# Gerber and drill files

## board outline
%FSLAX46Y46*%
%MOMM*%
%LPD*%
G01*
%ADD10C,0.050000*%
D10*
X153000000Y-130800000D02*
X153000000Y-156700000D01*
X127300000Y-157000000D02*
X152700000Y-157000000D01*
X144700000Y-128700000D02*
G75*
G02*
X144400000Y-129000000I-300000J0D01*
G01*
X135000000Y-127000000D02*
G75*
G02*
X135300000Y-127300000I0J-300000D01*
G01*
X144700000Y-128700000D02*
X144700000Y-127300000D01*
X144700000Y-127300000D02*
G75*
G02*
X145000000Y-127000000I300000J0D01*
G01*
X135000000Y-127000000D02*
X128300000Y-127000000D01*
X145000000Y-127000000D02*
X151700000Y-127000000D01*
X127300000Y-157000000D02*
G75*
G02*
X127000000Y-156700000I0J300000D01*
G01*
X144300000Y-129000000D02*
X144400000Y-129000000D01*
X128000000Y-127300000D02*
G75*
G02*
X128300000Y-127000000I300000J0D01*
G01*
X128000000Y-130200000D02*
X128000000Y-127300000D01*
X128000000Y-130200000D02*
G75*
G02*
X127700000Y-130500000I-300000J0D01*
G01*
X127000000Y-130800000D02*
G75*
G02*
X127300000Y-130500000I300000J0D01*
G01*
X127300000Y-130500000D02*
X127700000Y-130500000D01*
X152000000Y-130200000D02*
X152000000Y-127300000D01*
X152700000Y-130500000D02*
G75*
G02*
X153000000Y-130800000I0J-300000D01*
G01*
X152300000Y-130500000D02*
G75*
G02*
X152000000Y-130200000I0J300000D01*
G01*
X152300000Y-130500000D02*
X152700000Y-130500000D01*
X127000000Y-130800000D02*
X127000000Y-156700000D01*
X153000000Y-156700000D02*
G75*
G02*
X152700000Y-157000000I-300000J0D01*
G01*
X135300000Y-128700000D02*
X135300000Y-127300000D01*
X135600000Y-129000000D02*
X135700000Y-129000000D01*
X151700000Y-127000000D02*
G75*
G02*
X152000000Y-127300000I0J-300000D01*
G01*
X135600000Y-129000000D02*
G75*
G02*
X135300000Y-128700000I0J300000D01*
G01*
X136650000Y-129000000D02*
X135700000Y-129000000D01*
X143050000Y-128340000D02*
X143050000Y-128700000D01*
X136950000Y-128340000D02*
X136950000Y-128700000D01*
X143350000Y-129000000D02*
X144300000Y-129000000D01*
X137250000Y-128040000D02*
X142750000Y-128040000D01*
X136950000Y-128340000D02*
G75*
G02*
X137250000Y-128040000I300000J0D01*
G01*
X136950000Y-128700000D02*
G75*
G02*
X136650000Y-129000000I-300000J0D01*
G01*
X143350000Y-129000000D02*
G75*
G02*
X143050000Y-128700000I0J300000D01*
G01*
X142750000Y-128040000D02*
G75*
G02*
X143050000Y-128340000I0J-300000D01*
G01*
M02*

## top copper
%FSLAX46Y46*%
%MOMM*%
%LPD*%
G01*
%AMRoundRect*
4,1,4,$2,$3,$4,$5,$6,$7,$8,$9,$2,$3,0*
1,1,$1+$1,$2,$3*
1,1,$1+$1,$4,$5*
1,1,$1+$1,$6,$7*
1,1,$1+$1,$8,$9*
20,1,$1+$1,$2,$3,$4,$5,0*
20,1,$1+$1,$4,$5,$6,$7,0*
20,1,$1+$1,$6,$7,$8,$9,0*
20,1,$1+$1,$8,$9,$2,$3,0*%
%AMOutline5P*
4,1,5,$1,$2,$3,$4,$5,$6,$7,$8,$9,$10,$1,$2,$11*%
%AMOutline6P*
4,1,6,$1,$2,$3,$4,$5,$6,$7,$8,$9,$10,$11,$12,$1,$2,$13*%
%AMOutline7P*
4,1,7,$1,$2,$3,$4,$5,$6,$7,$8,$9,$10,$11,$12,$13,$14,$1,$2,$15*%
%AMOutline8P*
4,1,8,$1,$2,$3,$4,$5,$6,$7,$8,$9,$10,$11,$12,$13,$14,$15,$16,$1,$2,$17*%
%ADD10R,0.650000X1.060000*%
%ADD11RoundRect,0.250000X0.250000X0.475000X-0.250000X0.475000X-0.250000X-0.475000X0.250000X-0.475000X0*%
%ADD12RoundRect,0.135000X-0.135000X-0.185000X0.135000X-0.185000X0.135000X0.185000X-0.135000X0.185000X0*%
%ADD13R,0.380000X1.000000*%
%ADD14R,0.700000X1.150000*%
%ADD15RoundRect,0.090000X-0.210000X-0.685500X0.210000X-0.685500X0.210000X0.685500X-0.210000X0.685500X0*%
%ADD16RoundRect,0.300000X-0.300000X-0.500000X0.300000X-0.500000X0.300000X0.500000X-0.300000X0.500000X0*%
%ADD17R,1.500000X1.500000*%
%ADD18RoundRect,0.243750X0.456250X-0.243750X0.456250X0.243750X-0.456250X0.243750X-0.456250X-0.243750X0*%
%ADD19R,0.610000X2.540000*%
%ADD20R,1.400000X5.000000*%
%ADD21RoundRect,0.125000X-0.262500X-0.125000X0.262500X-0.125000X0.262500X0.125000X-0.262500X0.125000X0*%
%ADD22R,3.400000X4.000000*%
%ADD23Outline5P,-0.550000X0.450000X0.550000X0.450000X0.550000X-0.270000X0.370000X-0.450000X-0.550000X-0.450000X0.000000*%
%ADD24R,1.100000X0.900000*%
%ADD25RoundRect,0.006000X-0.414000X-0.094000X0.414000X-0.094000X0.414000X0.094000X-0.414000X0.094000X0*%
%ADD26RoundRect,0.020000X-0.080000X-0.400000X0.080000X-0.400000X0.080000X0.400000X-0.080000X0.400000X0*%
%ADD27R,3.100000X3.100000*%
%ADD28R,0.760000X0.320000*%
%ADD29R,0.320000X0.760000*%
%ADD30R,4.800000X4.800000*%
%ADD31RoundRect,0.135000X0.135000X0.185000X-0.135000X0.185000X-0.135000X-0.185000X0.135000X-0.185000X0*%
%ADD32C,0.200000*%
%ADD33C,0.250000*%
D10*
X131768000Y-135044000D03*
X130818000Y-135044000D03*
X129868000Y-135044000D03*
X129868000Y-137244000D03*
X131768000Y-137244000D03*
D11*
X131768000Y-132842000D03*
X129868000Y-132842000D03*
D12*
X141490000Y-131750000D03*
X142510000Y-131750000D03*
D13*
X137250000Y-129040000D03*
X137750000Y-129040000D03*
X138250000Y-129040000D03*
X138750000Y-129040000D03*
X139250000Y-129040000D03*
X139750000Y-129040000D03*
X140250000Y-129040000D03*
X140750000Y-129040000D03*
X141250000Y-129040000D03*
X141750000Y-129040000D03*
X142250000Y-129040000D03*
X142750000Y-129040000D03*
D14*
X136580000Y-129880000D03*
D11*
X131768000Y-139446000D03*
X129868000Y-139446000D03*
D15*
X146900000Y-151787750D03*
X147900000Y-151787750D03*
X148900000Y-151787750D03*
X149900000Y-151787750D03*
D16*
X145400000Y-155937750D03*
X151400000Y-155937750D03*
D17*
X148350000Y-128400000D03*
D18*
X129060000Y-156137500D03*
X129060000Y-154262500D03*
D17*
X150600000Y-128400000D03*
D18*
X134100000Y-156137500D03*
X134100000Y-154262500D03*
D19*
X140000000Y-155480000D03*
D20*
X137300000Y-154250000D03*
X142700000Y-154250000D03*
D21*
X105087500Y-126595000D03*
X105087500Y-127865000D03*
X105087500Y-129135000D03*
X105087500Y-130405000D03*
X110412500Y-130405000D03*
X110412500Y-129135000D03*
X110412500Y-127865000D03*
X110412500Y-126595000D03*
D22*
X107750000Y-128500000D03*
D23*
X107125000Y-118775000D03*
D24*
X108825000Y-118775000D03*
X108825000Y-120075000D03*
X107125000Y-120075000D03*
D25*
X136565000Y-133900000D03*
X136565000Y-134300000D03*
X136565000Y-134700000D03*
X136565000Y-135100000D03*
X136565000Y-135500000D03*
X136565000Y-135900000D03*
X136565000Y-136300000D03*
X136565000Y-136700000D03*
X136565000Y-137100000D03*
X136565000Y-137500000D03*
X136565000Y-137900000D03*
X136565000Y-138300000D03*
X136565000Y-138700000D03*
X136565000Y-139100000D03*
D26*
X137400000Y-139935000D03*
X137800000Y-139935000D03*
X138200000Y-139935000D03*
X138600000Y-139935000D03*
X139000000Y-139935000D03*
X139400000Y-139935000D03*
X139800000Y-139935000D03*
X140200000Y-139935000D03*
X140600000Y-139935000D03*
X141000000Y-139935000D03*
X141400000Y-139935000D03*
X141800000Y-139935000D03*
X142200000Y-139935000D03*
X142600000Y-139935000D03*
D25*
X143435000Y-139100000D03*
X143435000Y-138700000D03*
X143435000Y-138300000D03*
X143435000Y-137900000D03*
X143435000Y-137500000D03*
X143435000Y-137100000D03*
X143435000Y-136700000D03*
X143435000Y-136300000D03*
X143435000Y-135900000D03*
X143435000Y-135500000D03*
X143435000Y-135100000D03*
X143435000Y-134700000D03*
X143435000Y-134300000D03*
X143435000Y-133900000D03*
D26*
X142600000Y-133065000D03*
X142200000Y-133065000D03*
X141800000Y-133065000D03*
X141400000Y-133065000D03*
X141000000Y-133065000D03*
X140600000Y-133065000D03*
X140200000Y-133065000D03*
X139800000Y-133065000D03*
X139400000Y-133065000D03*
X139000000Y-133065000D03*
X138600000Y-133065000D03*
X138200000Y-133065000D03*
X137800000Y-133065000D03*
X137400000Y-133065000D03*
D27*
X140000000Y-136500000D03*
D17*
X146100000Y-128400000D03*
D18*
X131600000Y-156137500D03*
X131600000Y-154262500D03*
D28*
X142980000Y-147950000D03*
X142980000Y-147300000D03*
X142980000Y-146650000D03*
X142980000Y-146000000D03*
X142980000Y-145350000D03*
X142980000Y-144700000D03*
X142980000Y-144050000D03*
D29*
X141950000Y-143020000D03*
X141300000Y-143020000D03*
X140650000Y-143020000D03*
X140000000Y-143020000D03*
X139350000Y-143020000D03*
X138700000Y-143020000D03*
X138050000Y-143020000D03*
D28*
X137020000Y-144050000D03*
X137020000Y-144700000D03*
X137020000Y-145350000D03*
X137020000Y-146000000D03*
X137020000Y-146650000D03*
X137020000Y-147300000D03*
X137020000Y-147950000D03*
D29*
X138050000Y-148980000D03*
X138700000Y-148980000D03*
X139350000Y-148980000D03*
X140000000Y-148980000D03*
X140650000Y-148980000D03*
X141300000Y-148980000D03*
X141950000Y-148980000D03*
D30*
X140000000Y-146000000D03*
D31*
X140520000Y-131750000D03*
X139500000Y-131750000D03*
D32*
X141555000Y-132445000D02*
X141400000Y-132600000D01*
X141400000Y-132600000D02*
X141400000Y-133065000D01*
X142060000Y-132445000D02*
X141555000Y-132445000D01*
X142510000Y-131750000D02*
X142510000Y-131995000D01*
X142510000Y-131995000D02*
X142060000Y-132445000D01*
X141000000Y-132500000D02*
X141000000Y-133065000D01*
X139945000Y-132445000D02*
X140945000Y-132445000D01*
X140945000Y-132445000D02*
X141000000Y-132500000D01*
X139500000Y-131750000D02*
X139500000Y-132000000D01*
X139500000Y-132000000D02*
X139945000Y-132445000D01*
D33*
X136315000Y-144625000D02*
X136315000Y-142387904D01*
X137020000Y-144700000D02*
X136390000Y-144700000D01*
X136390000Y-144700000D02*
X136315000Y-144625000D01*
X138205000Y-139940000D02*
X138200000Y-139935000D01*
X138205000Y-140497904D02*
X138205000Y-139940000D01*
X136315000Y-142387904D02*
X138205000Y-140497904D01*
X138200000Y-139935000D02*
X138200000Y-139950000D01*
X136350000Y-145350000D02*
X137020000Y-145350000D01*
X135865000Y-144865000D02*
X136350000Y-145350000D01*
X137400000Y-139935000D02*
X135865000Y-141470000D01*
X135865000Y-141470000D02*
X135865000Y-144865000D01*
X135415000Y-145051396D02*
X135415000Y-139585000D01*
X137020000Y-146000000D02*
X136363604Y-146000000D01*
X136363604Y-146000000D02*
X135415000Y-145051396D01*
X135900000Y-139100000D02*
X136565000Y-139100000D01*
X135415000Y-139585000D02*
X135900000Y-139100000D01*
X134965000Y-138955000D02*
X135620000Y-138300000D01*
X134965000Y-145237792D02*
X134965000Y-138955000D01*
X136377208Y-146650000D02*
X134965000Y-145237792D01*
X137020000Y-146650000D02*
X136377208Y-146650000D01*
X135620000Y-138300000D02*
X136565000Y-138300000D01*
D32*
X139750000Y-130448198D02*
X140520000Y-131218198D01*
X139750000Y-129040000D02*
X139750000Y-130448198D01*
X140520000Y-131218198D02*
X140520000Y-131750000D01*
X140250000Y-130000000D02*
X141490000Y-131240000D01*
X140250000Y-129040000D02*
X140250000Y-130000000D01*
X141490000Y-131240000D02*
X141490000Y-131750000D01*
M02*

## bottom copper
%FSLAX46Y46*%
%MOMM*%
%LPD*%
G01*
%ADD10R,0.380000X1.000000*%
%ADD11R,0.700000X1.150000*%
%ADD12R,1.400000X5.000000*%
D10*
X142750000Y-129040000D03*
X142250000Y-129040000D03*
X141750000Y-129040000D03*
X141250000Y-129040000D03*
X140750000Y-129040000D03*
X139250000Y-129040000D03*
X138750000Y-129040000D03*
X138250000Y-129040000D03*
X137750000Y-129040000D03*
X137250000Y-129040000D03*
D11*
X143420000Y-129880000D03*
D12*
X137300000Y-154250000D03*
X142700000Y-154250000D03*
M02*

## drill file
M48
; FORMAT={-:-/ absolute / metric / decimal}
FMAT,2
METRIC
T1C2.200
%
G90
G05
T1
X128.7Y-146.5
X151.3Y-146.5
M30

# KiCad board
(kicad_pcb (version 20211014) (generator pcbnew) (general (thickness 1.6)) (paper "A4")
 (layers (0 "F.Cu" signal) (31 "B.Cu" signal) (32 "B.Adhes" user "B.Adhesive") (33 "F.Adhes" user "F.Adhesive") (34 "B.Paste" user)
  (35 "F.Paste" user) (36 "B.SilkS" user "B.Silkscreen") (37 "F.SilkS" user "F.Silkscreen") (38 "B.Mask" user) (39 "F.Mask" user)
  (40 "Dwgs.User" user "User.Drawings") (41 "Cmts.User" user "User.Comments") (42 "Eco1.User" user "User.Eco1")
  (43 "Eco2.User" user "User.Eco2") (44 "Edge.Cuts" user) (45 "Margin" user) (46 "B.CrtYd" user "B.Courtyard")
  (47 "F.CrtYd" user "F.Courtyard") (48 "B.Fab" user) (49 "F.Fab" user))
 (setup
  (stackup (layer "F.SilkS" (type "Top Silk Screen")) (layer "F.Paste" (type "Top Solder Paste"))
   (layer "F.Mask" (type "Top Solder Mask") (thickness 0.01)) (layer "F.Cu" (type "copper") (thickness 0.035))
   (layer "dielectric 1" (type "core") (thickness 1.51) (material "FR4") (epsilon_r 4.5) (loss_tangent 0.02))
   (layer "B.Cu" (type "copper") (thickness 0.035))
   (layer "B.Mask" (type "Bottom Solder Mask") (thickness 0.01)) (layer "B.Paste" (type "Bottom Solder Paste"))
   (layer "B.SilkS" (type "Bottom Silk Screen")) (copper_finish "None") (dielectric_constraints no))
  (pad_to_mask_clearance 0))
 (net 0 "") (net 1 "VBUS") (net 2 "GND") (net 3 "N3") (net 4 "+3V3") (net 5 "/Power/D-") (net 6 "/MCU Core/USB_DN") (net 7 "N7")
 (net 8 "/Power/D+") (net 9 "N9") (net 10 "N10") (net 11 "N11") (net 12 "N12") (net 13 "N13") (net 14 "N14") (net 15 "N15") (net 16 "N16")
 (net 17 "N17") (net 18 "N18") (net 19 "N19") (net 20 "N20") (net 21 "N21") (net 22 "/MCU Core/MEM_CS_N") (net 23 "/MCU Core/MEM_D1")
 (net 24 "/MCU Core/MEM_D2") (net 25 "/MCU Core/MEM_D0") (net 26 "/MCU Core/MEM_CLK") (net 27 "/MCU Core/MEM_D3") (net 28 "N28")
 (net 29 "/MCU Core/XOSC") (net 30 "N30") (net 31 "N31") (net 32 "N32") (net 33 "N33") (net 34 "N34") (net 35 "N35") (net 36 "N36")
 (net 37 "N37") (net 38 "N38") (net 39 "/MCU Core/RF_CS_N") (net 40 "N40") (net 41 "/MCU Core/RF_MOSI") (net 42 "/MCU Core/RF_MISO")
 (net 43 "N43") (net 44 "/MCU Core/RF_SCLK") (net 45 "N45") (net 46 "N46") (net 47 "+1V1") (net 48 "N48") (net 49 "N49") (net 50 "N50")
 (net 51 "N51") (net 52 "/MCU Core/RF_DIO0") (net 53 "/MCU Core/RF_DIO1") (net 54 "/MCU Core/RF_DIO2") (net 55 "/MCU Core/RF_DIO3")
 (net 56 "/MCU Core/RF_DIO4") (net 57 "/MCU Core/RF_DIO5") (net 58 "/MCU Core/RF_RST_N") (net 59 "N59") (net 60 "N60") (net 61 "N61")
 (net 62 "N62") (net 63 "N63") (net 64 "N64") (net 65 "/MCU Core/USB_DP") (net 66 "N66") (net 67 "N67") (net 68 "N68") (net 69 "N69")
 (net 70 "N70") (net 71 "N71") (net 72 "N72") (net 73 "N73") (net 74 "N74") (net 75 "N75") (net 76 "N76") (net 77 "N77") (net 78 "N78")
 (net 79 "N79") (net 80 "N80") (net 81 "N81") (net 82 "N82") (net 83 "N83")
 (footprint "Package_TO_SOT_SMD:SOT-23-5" (layer "F.Cu") (at 130.818 136.144 -90)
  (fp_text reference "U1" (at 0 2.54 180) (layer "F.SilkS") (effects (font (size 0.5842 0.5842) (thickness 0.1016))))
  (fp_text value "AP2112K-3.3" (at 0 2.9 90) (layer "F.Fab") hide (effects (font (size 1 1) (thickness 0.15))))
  (pad "1" smd rect locked (at -1.1 -0.95 270) (size 1.06 0.65) (layers "F.Cu" "F.Paste" "F.Mask") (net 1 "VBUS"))
  (pad "2" smd rect locked (at -1.1 0 270) (size 1.06 0.65) (layers "F.Cu" "F.Paste" "F.Mask") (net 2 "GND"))
  (pad "3" smd rect locked (at -1.1 0.95 270) (size 1.06 0.65) (layers "F.Cu" "F.Paste" "F.Mask") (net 1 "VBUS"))
  (pad "4" smd rect locked (at 1.1 0.95 270) (size 1.06 0.65) (layers "F.Cu" "F.Paste" "F.Mask") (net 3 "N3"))
  (pad "5" smd rect locked (at 1.1 -0.95 270) (size 1.06 0.65) (layers "F.Cu" "F.Paste" "F.Mask") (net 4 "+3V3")))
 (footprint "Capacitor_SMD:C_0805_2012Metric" (layer "F.Cu") (at 130.818 132.842 180)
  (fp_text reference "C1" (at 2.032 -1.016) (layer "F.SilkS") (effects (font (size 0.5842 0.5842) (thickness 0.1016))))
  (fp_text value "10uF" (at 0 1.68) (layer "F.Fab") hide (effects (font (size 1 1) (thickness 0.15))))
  (pad "1" smd roundrect locked (at -0.95 0 180) (size 1 1.45) (layers "F.Cu" "F.Paste" "F.Mask") (roundrect_rratio 0.25) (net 1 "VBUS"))
  (pad "2" smd roundrect locked (at 0.95 0 180) (size 1 1.45) (layers "F.Cu" "F.Paste" "F.Mask") (roundrect_rratio 0.25) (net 2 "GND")))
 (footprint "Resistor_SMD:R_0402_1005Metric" (layer "F.Cu") (at 142 131.75)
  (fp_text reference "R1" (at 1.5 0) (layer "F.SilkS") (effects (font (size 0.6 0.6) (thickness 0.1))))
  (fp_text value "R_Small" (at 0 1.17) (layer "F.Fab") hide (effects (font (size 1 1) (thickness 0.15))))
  (pad "1" smd roundrect (at -0.51 0) (size 0.54 0.64) (layers "F.Cu" "F.Paste" "F.Mask") (roundrect_rratio 0.25) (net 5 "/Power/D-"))
  (pad "2" smd roundrect (at 0.51 0) (size 0.54 0.64) (layers "F.Cu" "F.Paste" "F.Mask") (roundrect_rratio 0.25) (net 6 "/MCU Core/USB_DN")))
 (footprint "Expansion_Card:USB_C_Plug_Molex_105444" (layer "F.Cu") (at 140 129) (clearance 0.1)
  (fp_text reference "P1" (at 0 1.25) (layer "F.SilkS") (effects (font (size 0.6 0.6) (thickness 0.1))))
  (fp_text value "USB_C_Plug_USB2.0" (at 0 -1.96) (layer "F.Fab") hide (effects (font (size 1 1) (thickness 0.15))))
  (fp_line (start -3.35 0) (end -4.3 0) (layer "Edge.Cuts") (width 0.05))
  (fp_line (start 3.05 -0.66) (end 3.05 -0.3) (layer "Edge.Cuts") (width 0.05))
  (fp_line (start -3.05 -0.66) (end -3.05 -0.3) (layer "Edge.Cuts") (width 0.05))
  (fp_line (start 3.35 0) (end 4.3 0) (layer "Edge.Cuts") (width 0.05))
  (fp_line (start -2.75 -0.96) (end 2.75 -0.96) (layer "Edge.Cuts") (width 0.05))
  (fp_arc (start -3.05 -0.66) (mid -2.962132 -0.872132) (end -2.75 -0.96) (layer "Edge.Cuts") (width 0.05))
  (fp_arc (start -3.05 -0.3) (mid -3.137868 -0.087868) (end -3.35 0) (layer "Edge.Cuts") (width 0.05))
  (fp_arc (start 3.35 0) (mid 3.137868 -0.087868) (end 3.05 -0.3) (layer "Edge.Cuts") (width 0.05))
  (fp_arc (start 2.75 -0.96) (mid 2.962132 -0.872132) (end 3.05 -0.66) (layer "Edge.Cuts") (width 0.05))
  (pad "A1" smd rect locked (at -2.75 0.04) (size 0.38 1) (layers "F.Cu" "F.Paste" "F.Mask") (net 2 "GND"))
  (pad "A2" smd rect locked (at -2.25 0.04) (size 0.38 1) (layers "F.Cu" "F.Paste" "F.Mask"))
  (pad "A3" smd rect locked (at -1.75 0.04) (size 0.38 1) (layers "F.Cu" "F.Paste" "F.Mask"))
  (pad "A4" smd rect locked (at -1.25 0.04) (size 0.38 1) (layers "F.Cu" "F.Paste" "F.Mask") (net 1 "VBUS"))
  (pad "A5" smd rect locked (at -0.75 0.04) (size 0.38 1) (layers "F.Cu" "F.Paste" "F.Mask") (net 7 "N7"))
  (pad "A6" smd rect locked (at -0.25 0.04) (size 0.38 1) (layers "F.Cu" "F.Paste" "F.Mask") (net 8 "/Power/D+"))
  (pad "A7" smd rect locked (at 0.25 0.04) (size 0.38 1) (layers "F.Cu" "F.Paste" "F.Mask") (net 5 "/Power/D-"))
  (pad "A8" smd rect locked (at 0.75 0.04) (size 0.38 1) (layers "F.Cu" "F.Paste" "F.Mask"))
  (pad "A9" smd rect locked (at 1.25 0.04) (size 0.38 1) (layers "F.Cu" "F.Paste" "F.Mask") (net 1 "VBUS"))
  (pad "A10" smd rect locked (at 1.75 0.04) (size 0.38 1) (layers "F.Cu" "F.Paste" "F.Mask"))
  (pad "A11" smd rect locked (at 2.25 0.04) (size 0.38 1) (layers "F.Cu" "F.Paste" "F.Mask"))
  (pad "A12" smd rect locked (at 2.75 0.04) (size 0.38 1) (layers "F.Cu" "F.Paste" "F.Mask") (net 2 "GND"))
  (pad "B1" smd rect locked (at 2.75 0.04) (size 0.38 1) (layers "B.Cu" "B.Paste" "B.Mask") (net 2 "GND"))
  (pad "B2" smd rect locked (at 2.25 0.04) (size 0.38 1) (layers "B.Cu" "B.Paste" "B.Mask"))
  (pad "B3" smd rect locked (at 1.75 0.04) (size 0.38 1) (layers "B.Cu" "B.Paste" "B.Mask"))
  (pad "B4" smd rect locked (at 1.25 0.04) (size 0.38 1) (layers "B.Cu" "B.Paste" "B.Mask") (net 1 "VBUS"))
  (pad "B5" smd rect locked (at 0.75 0.04) (size 0.38 1) (layers "B.Cu" "B.Paste" "B.Mask") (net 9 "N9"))
  (pad "B8" smd rect locked (at -0.75 0.04) (size 0.38 1) (layers "B.Cu" "B.Paste" "B.Mask"))
  (pad "B9" smd rect locked (at -1.25 0.04) (size 0.38 1) (layers "B.Cu" "B.Paste" "B.Mask") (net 1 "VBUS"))
  (pad "B10" smd rect locked (at -1.75 0.04) (size 0.38 1) (layers "B.Cu" "B.Paste" "B.Mask"))
  (pad "B11" smd rect locked (at -2.25 0.04) (size 0.38 1) (layers "B.Cu" "B.Paste" "B.Mask"))
  (pad "B12" smd rect locked (at -2.75 0.04) (size 0.38 1) (layers "B.Cu" "B.Paste" "B.Mask") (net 2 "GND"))
  (pad "S1" smd rect locked (at -3.42 0.88) (size 0.7 1.15) (layers "F.Cu" "F.Paste" "F.Mask") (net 2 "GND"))
  (pad "S1" smd rect locked (at 3.42 0.88) (size 0.7 1.15) (layers "B.Cu" "B.Paste" "B.Mask") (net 2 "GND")))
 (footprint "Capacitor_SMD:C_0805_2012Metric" (layer "F.Cu") (at 130.818 139.446 180)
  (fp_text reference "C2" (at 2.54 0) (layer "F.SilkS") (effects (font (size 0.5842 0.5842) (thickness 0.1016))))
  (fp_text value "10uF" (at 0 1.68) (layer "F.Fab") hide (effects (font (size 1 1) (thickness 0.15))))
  (pad "1" smd roundrect locked (at -0.95 0 180) (size 1 1.45) (layers "F.Cu" "F.Paste" "F.Mask") (roundrect_rratio 0.25) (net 4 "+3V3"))
  (pad "2" smd roundrect locked (at 0.95 0 180) (size 1 1.45) (layers "F.Cu" "F.Paste" "F.Mask") (roundrect_rratio 0.25) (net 2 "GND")))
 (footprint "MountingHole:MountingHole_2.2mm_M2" (layer "F.Cu") (at 128.7 146.5)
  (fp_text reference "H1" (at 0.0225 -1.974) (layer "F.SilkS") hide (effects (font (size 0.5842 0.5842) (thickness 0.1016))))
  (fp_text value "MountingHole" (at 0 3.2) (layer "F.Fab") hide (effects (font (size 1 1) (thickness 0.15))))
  (pad "" np_thru_hole circle locked (at 0 0) (size 2.2 2.2) (drill 2.2) (layers *.Cu *.Mask)))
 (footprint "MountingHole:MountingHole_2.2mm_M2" (layer "F.Cu") (at 151.3 146.5)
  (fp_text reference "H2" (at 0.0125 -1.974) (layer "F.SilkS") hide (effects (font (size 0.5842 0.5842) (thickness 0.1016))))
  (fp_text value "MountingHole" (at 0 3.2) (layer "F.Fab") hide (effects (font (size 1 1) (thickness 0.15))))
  (pad "" np_thru_hole circle locked (at 0 0) (size 2.2 2.2) (drill 2.2) (layers *.Cu *.Mask)))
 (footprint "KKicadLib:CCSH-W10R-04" (layer "F.Cu") (at 148.4 151.78775)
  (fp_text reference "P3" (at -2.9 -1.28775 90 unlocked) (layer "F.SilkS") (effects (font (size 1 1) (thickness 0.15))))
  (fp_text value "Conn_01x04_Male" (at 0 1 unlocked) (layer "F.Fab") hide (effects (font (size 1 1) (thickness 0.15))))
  (pad "1" smd roundrect (at -1.5 0) (size 0.6 1.551) (layers "F.Cu" "F.Paste" "F.Mask") (roundrect_rratio 0.15) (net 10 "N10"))
  (pad "2" smd roundrect (at -0.5 0) (size 0.6 1.551) (layers "F.Cu" "F.Paste" "F.Mask") (roundrect_rratio 0.15) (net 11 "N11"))
  (pad "3" smd roundrect (at 0.5 0) (size 0.6 1.551) (layers "F.Cu" "F.Paste" "F.Mask") (roundrect_rratio 0.15) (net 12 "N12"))
  (pad "4" smd roundrect (at 1.5 0) (size 0.6 1.551) (layers "F.Cu" "F.Paste" "F.Mask") (roundrect_rratio 0.15) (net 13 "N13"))
  (pad "MECH" smd roundrect (at -3 4.15) (size 1.2 1.6) (layers "F.Cu" "F.Paste" "F.Mask") (roundrect_rratio 0.25))
  (pad "MECH" smd roundrect (at 3 4.15) (size 1.2 1.6) (layers "F.Cu" "F.Paste" "F.Mask") (roundrect_rratio 0.25))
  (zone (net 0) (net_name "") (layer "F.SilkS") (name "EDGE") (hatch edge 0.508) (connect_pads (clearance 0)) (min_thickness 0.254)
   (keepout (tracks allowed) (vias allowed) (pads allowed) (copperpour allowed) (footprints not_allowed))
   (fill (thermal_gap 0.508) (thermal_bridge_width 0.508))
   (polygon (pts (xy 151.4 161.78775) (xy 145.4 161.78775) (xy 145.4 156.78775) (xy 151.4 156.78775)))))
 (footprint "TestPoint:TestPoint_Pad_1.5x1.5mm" (layer "F.Cu") (at 148.35 128.4)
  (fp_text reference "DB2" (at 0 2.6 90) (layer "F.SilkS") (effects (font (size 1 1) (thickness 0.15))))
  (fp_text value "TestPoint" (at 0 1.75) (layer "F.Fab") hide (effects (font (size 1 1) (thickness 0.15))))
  (pad "1" smd rect (at 0 0) (size 1.5 1.5) (layers "F.Cu" "F.Mask") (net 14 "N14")))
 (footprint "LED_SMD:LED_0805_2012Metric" (layer "F.Cu") (at 129.06 155.2 90)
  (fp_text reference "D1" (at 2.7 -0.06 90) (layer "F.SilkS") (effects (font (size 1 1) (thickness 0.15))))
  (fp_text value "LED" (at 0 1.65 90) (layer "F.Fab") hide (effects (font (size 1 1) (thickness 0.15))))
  (pad "1" smd roundrect (at -0.9375 0 90) (size 0.975 1.4) (layers "F.Cu" "F.Paste" "F.Mask") (roundrect_rratio 0.25) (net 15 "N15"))
  (pad "2" smd roundrect (at 0.9375 0 90) (size 0.975 1.4) (layers "F.Cu" "F.Paste" "F.Mask") (roundrect_rratio 0.25) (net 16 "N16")))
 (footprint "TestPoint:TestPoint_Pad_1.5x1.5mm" (layer "F.Cu") (at 150.6 128.4)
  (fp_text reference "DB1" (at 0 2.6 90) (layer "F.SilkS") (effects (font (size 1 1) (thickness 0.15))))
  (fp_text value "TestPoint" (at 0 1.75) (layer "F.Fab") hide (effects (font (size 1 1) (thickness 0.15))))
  (pad "1" smd rect (at 0 0) (size 1.5 1.5) (layers "F.Cu" "F.Mask") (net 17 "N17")))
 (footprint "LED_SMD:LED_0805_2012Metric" (layer "F.Cu") (at 134.1 155.2 90)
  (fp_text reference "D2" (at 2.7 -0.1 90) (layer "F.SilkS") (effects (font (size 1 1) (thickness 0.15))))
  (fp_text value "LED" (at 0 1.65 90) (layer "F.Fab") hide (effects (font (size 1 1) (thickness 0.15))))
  (pad "1" smd roundrect (at -0.9375 0 90) (size 0.975 1.4) (layers "F.Cu" "F.Paste" "F.Mask") (roundrect_rratio 0.25) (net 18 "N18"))
  (pad "2" smd roundrect (at 0.9375 0 90) (size 0.975 1.4) (layers "F.Cu" "F.Paste" "F.Mask") (roundrect_rratio 0.25) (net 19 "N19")))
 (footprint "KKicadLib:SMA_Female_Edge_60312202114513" (layer "F.Cu") (at 140 156.75)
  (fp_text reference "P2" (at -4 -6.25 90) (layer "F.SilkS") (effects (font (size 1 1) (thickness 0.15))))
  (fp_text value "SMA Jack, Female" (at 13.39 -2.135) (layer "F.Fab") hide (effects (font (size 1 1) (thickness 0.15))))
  (pad "1" smd rect (at 0 -1.27) (size 0.61 2.54) (layers "F.Cu" "F.Paste" "F.Mask") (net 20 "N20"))
  (pad "2" smd rect (at -2.7 -2.5) (size 1.4 5) (layers "F.Cu" "F.Paste" "F.Mask") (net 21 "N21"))
  (pad "3" smd rect (at 2.7 -2.5) (size 1.4 5) (layers "F.Cu" "F.Paste" "F.Mask") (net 21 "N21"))
  (pad "4" smd rect (at -2.7 -2.5) (size 1.4 5) (layers "B.Cu" "B.Paste" "B.Mask") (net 21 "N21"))
  (pad "5" smd rect (at 2.7 -2.5) (size 1.4 5) (layers "B.Cu" "B.Paste" "B.Mask") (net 21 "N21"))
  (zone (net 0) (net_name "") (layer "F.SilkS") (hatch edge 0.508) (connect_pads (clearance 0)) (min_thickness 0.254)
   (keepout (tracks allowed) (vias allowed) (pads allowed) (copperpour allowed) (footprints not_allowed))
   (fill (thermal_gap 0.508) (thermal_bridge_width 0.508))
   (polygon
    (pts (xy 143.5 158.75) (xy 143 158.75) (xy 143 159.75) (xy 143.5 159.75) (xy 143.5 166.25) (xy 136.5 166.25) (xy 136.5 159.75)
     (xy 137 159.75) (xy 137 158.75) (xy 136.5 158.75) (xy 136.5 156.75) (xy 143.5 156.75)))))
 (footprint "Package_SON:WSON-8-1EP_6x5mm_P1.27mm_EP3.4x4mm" (layer "F.Cu") (at 107.75 128.5)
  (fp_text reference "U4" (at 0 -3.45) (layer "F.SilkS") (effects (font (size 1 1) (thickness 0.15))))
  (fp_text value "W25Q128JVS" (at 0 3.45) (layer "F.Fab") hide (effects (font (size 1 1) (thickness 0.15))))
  (pad "" smd roundrect (at 0.85 -1) (size 1.37 1.61) (layers "F.Paste") (roundrect_rratio 0.182482))
  (pad "" smd roundrect (at -0.85 -1) (size 1.37 1.61) (layers "F.Paste") (roundrect_rratio 0.182482))
  (pad "" smd roundrect (at -0.85 1) (size 1.37 1.61) (layers "F.Paste") (roundrect_rratio 0.182482))
  (pad "" smd roundrect (at 0.85 1) (size 1.37 1.61) (layers "F.Paste") (roundrect_rratio 0.182482))
  (pad "1" smd roundrect (at -2.6625 -1.905) (size 0.775 0.5) (layers "F.Cu" "F.Paste" "F.Mask") (roundrect_rratio 0.25)
   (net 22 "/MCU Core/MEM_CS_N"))
  (pad "2" smd roundrect (at -2.6625 -0.635) (size 0.775 0.5) (layers "F.Cu" "F.Paste" "F.Mask") (roundrect_rratio 0.25)
   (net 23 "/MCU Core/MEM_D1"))
  (pad "3" smd roundrect (at -2.6625 0.635) (size 0.775 0.5) (layers "F.Cu" "F.Paste" "F.Mask") (roundrect_rratio 0.25)
   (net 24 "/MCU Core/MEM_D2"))
  (pad "4" smd roundrect (at -2.6625 1.905) (size 0.775 0.5) (layers "F.Cu" "F.Paste" "F.Mask") (roundrect_rratio 0.25) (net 2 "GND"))
  (pad "5" smd roundrect (at 2.6625 1.905) (size 0.775 0.5) (layers "F.Cu" "F.Paste" "F.Mask") (roundrect_rratio 0.25)
   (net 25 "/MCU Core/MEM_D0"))
  (pad "6" smd roundrect (at 2.6625 0.635) (size 0.775 0.5) (layers "F.Cu" "F.Paste" "F.Mask") (roundrect_rratio 0.25)
   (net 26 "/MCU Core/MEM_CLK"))
  (pad "7" smd roundrect (at 2.6625 -0.635) (size 0.775 0.5) (layers "F.Cu" "F.Paste" "F.Mask") (roundrect_rratio 0.25)
   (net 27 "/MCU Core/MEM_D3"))
  (pad "8" smd roundrect (at 2.6625 -1.905) (size 0.775 0.5) (layers "F.Cu" "F.Paste" "F.Mask") (roundrect_rratio 0.25) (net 4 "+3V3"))
  (pad "9" smd rect (at 0 0) (size 3.4 4) (layers "F.Cu" "F.Mask")))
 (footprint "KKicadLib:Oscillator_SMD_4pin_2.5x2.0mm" (layer "F.Cu") (at 107.975 119.425)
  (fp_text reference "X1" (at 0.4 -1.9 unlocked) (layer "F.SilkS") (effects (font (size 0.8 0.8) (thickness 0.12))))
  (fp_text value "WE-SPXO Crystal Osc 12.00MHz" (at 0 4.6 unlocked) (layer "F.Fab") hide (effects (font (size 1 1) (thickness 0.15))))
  (pad "1" smd roundrect (at -0.85 -0.65) (size 1.1 0.9) (layers "F.Cu" "F.Paste" "F.Mask") (roundrect_rratio 0) (chamfer_ratio 0.2)
   (chamfer bottom_right) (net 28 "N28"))
  (pad "2" smd rect (at 0.85 -0.65) (size 1.1 0.9) (layers "F.Cu" "F.Paste" "F.Mask") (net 2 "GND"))
  (pad "3" smd rect (at 0.85 0.65) (size 1.1 0.9) (layers "F.Cu" "F.Paste" "F.Mask") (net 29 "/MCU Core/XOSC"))
  (pad "4" smd rect (at -0.85 0.65) (size 1.1 0.9) (layers "F.Cu" "F.Paste" "F.Mask") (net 28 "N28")))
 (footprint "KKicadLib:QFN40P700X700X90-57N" (layer "F.Cu") (at 140 136.5) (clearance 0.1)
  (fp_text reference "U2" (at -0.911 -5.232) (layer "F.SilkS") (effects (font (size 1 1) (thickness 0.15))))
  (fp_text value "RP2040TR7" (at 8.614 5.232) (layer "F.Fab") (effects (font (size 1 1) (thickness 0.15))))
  (pad "1" smd roundrect (at -3.435 -2.6) (size 0.84 0.2) (layers "F.Cu" "F.Paste" "F.Mask") (roundrect_rratio 0.03) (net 4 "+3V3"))
  (pad "2" smd roundrect (at -3.435 -2.2) (size 0.84 0.2) (layers "F.Cu" "F.Paste" "F.Mask") (roundrect_rratio 0.03) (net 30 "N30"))
  (pad "3" smd roundrect (at -3.435 -1.8) (size 0.84 0.2) (layers "F.Cu" "F.Paste" "F.Mask") (roundrect_rratio 0.03) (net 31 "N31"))
  (pad "4" smd roundrect (at -3.435 -1.4) (size 0.84 0.2) (layers "F.Cu" "F.Paste" "F.Mask") (roundrect_rratio 0.03) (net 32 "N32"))
  (pad "5" smd roundrect (at -3.435 -1) (size 0.84 0.2) (layers "F.Cu" "F.Paste" "F.Mask") (roundrect_rratio 0.03) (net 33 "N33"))
  (pad "6" smd roundrect (at -3.435 -0.6) (size 0.84 0.2) (layers "F.Cu" "F.Paste" "F.Mask") (roundrect_rratio 0.03) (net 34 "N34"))
  (pad "7" smd roundrect (at -3.435 -0.2) (size 0.84 0.2) (layers "F.Cu" "F.Paste" "F.Mask") (roundrect_rratio 0.03) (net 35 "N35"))
  (pad "8" smd roundrect (at -3.435 0.2) (size 0.84 0.2) (layers "F.Cu" "F.Paste" "F.Mask") (roundrect_rratio 0.03) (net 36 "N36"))
  (pad "9" smd roundrect (at -3.435 0.6) (size 0.84 0.2) (layers "F.Cu" "F.Paste" "F.Mask") (roundrect_rratio 0.03) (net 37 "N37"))
  (pad "10" smd roundrect (at -3.435 1) (size 0.84 0.2) (layers "F.Cu" "F.Paste" "F.Mask") (roundrect_rratio 0.03) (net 4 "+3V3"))
  (pad "11" smd roundrect (at -3.435 1.4) (size 0.84 0.2) (layers "F.Cu" "F.Paste" "F.Mask") (roundrect_rratio 0.03) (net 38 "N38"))
  (pad "12" smd roundrect (at -3.435 1.8) (size 0.84 0.2) (layers "F.Cu" "F.Paste" "F.Mask") (roundrect_rratio 0.03)
   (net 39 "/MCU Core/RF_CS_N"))
  (pad "13" smd roundrect (at -3.435 2.2) (size 0.84 0.2) (layers "F.Cu" "F.Paste" "F.Mask") (roundrect_rratio 0.03) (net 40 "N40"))
  (pad "14" smd roundrect (at -3.435 2.6) (size 0.84 0.2) (layers "F.Cu" "F.Paste" "F.Mask") (roundrect_rratio 0.03)
   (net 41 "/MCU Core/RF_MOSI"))
  (pad "15" smd roundrect (at -2.6 3.435) (size 0.2 0.84) (layers "F.Cu" "F.Paste" "F.Mask") (roundrect_rratio 0.1)
   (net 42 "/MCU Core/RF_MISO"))
  (pad "16" smd roundrect (at -2.2 3.435) (size 0.2 0.84) (layers "F.Cu" "F.Paste" "F.Mask") (roundrect_rratio 0.1) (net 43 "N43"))
  (pad "17" smd roundrect (at -1.8 3.435) (size 0.2 0.84) (layers "F.Cu" "F.Paste" "F.Mask") (roundrect_rratio 0.1)
   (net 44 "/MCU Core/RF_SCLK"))
  (pad "18" smd roundrect (at -1.4 3.435) (size 0.2 0.84) (layers "F.Cu" "F.Paste" "F.Mask") (roundrect_rratio 0.1) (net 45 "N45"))
  (pad "19" smd roundrect (at -1 3.435) (size 0.2 0.84) (layers "F.Cu" "F.Paste" "F.Mask") (roundrect_rratio 0.1) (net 2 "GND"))
  (pad "20" smd roundrect (at -0.6 3.435) (size 0.2 0.84) (layers "F.Cu" "F.Paste" "F.Mask") (roundrect_rratio 0.1)
   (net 29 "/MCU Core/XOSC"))
  (pad "21" smd roundrect (at -0.2 3.435) (size 0.2 0.84) (layers "F.Cu" "F.Paste" "F.Mask") (roundrect_rratio 0.1) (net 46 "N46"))
  (pad "22" smd roundrect (at 0.2 3.435) (size 0.2 0.84) (layers "F.Cu" "F.Paste" "F.Mask") (roundrect_rratio 0.1) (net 4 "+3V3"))
  (pad "23" smd roundrect (at 0.6 3.435) (size 0.2 0.84) (layers "F.Cu" "F.Paste" "F.Mask") (roundrect_rratio 0.1) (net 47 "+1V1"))
  (pad "24" smd roundrect (at 1 3.435) (size 0.2 0.84) (layers "F.Cu" "F.Paste" "F.Mask") (roundrect_rratio 0.1) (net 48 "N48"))
  (pad "25" smd roundrect (at 1.4 3.435) (size 0.2 0.84) (layers "F.Cu" "F.Paste" "F.Mask") (roundrect_rratio 0.1) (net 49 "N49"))
  (pad "26" smd roundrect (at 1.8 3.435) (size 0.2 0.84) (layers "F.Cu" "F.Paste" "F.Mask") (roundrect_rratio 0.1) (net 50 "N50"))
  (pad "27" smd roundrect (at 2.2 3.435) (size 0.2 0.84) (layers "F.Cu" "F.Paste" "F.Mask") (roundrect_rratio 0.1) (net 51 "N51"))
  (pad "28" smd roundrect (at 2.6 3.435) (size 0.2 0.84) (layers "F.Cu" "F.Paste" "F.Mask") (roundrect_rratio 0.1)
   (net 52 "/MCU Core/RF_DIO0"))
  (pad "29" smd roundrect (at 3.435 2.6) (size 0.84 0.2) (layers "F.Cu" "F.Paste" "F.Mask") (roundrect_rratio 0.03)
   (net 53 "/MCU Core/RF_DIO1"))
  (pad "30" smd roundrect (at 3.435 2.2) (size 0.84 0.2) (layers "F.Cu" "F.Paste" "F.Mask") (roundrect_rratio 0.03)
   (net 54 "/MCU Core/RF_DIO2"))
  (pad "31" smd roundrect (at 3.435 1.8) (size 0.84 0.2) (layers "F.Cu" "F.Paste" "F.Mask") (roundrect_rratio 0.03)
   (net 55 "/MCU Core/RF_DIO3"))
  (pad "32" smd roundrect (at 3.435 1.4) (size 0.84 0.2) (layers "F.Cu" "F.Paste" "F.Mask") (roundrect_rratio 0.03)
   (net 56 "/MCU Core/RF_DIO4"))
  (pad "33" smd roundrect (at 3.435 1) (size 0.84 0.2) (layers "F.Cu" "F.Paste" "F.Mask") (roundrect_rratio 0.03) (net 4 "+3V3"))
  (pad "34" smd roundrect (at 3.435 0.6) (size 0.84 0.2) (layers "F.Cu" "F.Paste" "F.Mask") (roundrect_rratio 0.03)
   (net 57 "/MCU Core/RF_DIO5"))
  (pad "35" smd roundrect (at 3.435 0.2) (size 0.84 0.2) (layers "F.Cu" "F.Paste" "F.Mask") (roundrect_rratio 0.03)
   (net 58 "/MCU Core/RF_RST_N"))
  (pad "36" smd roundrect (at 3.435 -0.2) (size 0.84 0.2) (layers "F.Cu" "F.Paste" "F.Mask") (roundrect_rratio 0.03) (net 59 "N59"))
  (pad "37" smd roundrect (at 3.435 -0.6) (size 0.84 0.2) (layers "F.Cu" "F.Paste" "F.Mask") (roundrect_rratio 0.03) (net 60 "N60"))
  (pad "38" smd roundrect (at 3.435 -1) (size 0.84 0.2) (layers "F.Cu" "F.Paste" "F.Mask") (roundrect_rratio 0.03) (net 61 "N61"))
  (pad "39" smd roundrect (at 3.435 -1.4) (size 0.84 0.2) (layers "F.Cu" "F.Paste" "F.Mask") (roundrect_rratio 0.03) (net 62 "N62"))
  (pad "40" smd roundrect (at 3.435 -1.8) (size 0.84 0.2) (layers "F.Cu" "F.Paste" "F.Mask") (roundrect_rratio 0.03) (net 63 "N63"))
  (pad "41" smd roundrect (at 3.435 -2.2) (size 0.84 0.2) (layers "F.Cu" "F.Paste" "F.Mask") (roundrect_rratio 0.03) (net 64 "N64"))
  (pad "42" smd roundrect (at 3.435 -2.6) (size 0.84 0.2) (layers "F.Cu" "F.Paste" "F.Mask") (roundrect_rratio 0.03) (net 4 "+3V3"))
  (pad "43" smd roundrect (at 2.6 -3.435) (size 0.2 0.84) (layers "F.Cu" "F.Paste" "F.Mask") (roundrect_rratio 0.1) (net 4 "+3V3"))
  (pad "44" smd roundrect (at 2.2 -3.435) (size 0.2 0.84) (layers "F.Cu" "F.Paste" "F.Mask") (roundrect_rratio 0.1) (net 4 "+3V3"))
  (pad "45" smd roundrect (at 1.8 -3.435) (size 0.2 0.84) (layers "F.Cu" "F.Paste" "F.Mask") (roundrect_rratio 0.1) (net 47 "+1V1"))
  (pad "46" smd roundrect (at 1.4 -3.435) (size 0.2 0.84) (layers "F.Cu" "F.Paste" "F.Mask") (roundrect_rratio 0.1)
   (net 6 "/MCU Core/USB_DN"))
  (pad "47" smd roundrect (at 1 -3.435) (size 0.2 0.84) (layers "F.Cu" "F.Paste" "F.Mask") (roundrect_rratio 0.1)
   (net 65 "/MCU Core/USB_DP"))
  (pad "48" smd roundrect (at 0.6 -3.435) (size 0.2 0.84) (layers "F.Cu" "F.Paste" "F.Mask") (roundrect_rratio 0.1) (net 4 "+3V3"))
  (pad "49" smd roundrect (at 0.2 -3.435) (size 0.2 0.84) (layers "F.Cu" "F.Paste" "F.Mask") (roundrect_rratio 0.1) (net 4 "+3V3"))
  (pad "50" smd roundrect (at -0.2 -3.435) (size 0.2 0.84) (layers "F.Cu" "F.Paste" "F.Mask") (roundrect_rratio 0.1) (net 47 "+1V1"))
  (pad "51" smd roundrect (at -0.6 -3.435) (size 0.2 0.84) (layers "F.Cu" "F.Paste" "F.Mask") (roundrect_rratio 0.1)
   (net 27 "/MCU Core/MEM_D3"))
  (pad "52" smd roundrect (at -1 -3.435) (size 0.2 0.84) (layers "F.Cu" "F.Paste" "F.Mask") (roundrect_rratio 0.1)
   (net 26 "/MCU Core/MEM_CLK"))
  (pad "53" smd roundrect (at -1.4 -3.435) (size 0.2 0.84) (layers "F.Cu" "F.Paste" "F.Mask") (roundrect_rratio 0.1)
   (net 25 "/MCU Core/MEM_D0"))
  (pad "54" smd roundrect (at -1.8 -3.435) (size 0.2 0.84) (layers "F.Cu" "F.Paste" "F.Mask") (roundrect_rratio 0.1)
   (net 24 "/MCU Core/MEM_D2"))
  (pad "55" smd roundrect (at -2.2 -3.435) (size 0.2 0.84) (layers "F.Cu" "F.Paste" "F.Mask") (roundrect_rratio 0.1)
   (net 23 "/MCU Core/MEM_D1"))
  (pad "56" smd roundrect (at -2.6 -3.435) (size 0.2 0.84) (layers "F.Cu" "F.Paste" "F.Mask") (roundrect_rratio 0.1)
   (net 22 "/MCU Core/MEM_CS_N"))
  (pad "57" smd rect (at 0 0) (size 3.1 3.1) (layers "F.Cu" "F.Mask") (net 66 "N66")))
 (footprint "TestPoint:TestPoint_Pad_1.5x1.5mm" (layer "F.Cu") (at 146.1 128.4)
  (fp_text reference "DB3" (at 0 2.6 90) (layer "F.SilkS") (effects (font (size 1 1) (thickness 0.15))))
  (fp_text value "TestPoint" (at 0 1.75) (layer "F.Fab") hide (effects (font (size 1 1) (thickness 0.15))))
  (pad "1" smd rect (at 0 0) (size 1.5 1.5) (layers "F.Cu" "F.Mask") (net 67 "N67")))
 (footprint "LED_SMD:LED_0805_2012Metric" (layer "F.Cu") (at 131.6 155.2 90)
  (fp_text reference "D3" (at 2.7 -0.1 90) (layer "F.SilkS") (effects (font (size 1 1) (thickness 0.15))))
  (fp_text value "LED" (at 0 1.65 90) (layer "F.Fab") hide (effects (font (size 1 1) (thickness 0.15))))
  (pad "1" smd roundrect (at -0.9375 0 90) (size 0.975 1.4) (layers "F.Cu" "F.Paste" "F.Mask") (roundrect_rratio 0.25) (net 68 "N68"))
  (pad "2" smd roundrect (at 0.9375 0 90) (size 0.975 1.4) (layers "F.Cu" "F.Paste" "F.Mask") (roundrect_rratio 0.25) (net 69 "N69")))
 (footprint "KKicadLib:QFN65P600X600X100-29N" (layer "F.Cu") (at 140 146 180)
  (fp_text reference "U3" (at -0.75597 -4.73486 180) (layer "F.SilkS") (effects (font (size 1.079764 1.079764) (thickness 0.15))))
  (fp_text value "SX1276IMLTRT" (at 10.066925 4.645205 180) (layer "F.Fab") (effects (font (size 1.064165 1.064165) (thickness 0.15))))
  (pad "1" smd rect locked (at -2.98 -1.95 180) (size 0.76 0.32) (layers "F.Cu" "F.Paste" "F.Mask") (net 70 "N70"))
  (pad "2" smd rect locked (at -2.98 -1.3 180) (size 0.76 0.32) (layers "F.Cu" "F.Paste" "F.Mask") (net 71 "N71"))
  (pad "3" smd rect locked (at -2.98 -0.65 180) (size 0.76 0.32) (layers "F.Cu" "F.Paste" "F.Mask") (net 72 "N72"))
  (pad "4" smd rect locked (at -2.98 0 180) (size 0.76 0.32) (layers "F.Cu" "F.Paste" "F.Mask") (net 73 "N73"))
  (pad "5" smd rect locked (at -2.98 0.65 180) (size 0.76 0.32) (layers "F.Cu" "F.Paste" "F.Mask") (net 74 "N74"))
  (pad "6" smd rect locked (at -2.98 1.3 180) (size 0.76 0.32) (layers "F.Cu" "F.Paste" "F.Mask") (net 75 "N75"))
  (pad "7" smd rect locked (at -2.98 1.95 180) (size 0.76 0.32) (layers "F.Cu" "F.Paste" "F.Mask") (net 58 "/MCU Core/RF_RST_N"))
  (pad "8" smd rect locked (at -1.95 2.98 90) (size 0.76 0.32) (layers "F.Cu" "F.Paste" "F.Mask") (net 52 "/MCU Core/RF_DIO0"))
  (pad "9" smd rect locked (at -1.3 2.98 90) (size 0.76 0.32) (layers "F.Cu" "F.Paste" "F.Mask") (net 53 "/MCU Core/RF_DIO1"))
  (pad "10" smd rect locked (at -0.65 2.98 90) (size 0.76 0.32) (layers "F.Cu" "F.Paste" "F.Mask") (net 54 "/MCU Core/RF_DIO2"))
  (pad "11" smd rect locked (at 0 2.98 90) (size 0.76 0.32) (layers "F.Cu" "F.Paste" "F.Mask") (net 55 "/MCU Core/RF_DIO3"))
  (pad "12" smd rect locked (at 0.65 2.98 90) (size 0.76 0.32) (layers "F.Cu" "F.Paste" "F.Mask") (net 56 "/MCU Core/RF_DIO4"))
  (pad "13" smd rect locked (at 1.3 2.98 90) (size 0.76 0.32) (layers "F.Cu" "F.Paste" "F.Mask") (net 57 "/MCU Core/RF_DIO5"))
  (pad "14" smd rect locked (at 1.95 2.98 90) (size 0.76 0.32) (layers "F.Cu" "F.Paste" "F.Mask") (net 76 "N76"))
  (pad "15" smd rect locked (at 2.98 1.95) (size 0.76 0.32) (layers "F.Cu" "F.Paste" "F.Mask") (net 2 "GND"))
  (pad "16" smd rect locked (at 2.98 1.3) (size 0.76 0.32) (layers "F.Cu" "F.Paste" "F.Mask") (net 44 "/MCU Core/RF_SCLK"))
  (pad "17" smd rect locked (at 2.98 0.65) (size 0.76 0.32) (layers "F.Cu" "F.Paste" "F.Mask") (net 42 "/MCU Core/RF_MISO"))
  (pad "18" smd rect locked (at 2.98 0) (size 0.76 0.32) (layers "F.Cu" "F.Paste" "F.Mask") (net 41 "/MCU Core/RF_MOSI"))
  (pad "19" smd rect locked (at 2.98 -0.65) (size 0.76 0.32) (layers "F.Cu" "F.Paste" "F.Mask") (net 39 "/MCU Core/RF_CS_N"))
  (pad "20" smd rect locked (at 2.98 -1.3) (size 0.76 0.32) (layers "F.Cu" "F.Paste" "F.Mask") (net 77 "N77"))
  (pad "21" smd rect locked (at 2.98 -1.95) (size 0.76 0.32) (layers "F.Cu" "F.Paste" "F.Mask") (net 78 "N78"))
  (pad "22" smd rect locked (at 1.95 -2.98 270) (size 0.76 0.32) (layers "F.Cu" "F.Paste" "F.Mask") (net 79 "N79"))
  (pad "23" smd rect locked (at 1.3 -2.98 270) (size 0.76 0.32) (layers "F.Cu" "F.Paste" "F.Mask") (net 2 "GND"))
  (pad "24" smd rect locked (at 0.65 -2.98 270) (size 0.76 0.32) (layers "F.Cu" "F.Paste" "F.Mask") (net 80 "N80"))
  (pad "25" smd rect locked (at 0 -2.98 270) (size 0.76 0.32) (layers "F.Cu" "F.Paste" "F.Mask") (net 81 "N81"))
  (pad "26" smd rect locked (at -0.65 -2.98 270) (size 0.76 0.32) (layers "F.Cu" "F.Paste" "F.Mask") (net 2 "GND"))
  (pad "27" smd rect locked (at -1.3 -2.98 270) (size 0.76 0.32) (layers "F.Cu" "F.Paste" "F.Mask") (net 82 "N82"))
  (pad "28" smd rect locked (at -1.95 -2.98 270) (size 0.76 0.32) (layers "F.Cu" "F.Paste" "F.Mask") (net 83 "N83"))
  (pad "29" smd rect locked (at 0 0 180) (size 4.8 4.8) (layers "F.Cu" "F.Mask") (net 2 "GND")))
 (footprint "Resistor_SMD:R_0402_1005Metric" (layer "F.Cu") (at 140.01 131.75 180)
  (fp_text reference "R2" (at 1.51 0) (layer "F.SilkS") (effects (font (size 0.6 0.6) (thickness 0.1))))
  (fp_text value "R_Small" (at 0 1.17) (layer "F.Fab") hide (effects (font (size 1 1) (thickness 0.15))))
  (pad "1" smd roundrect (at -0.51 0 180) (size 0.54 0.64) (layers "F.Cu" "F.Paste" "F.Mask") (roundrect_rratio 0.25) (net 8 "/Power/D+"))
  (pad "2" smd roundrect (at 0.51 0 180) (size 0.54 0.64) (layers "F.Cu" "F.Paste" "F.Mask") (roundrect_rratio 0.25)
   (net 65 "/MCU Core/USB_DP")))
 (gr_line (start 153 130.8) (end 153 156.7) (layer "Edge.Cuts") (width 0.05))
 (gr_line (start 127.3 157) (end 152.7 157) (layer "Edge.Cuts") (width 0.05))
 (gr_arc (start 144.7 128.7) (mid 144.612132 128.912132) (end 144.4 129) (layer "Edge.Cuts") (width 0.05))
 (gr_arc (start 135 127) (mid 135.212132 127.087868) (end 135.3 127.3) (layer "Edge.Cuts") (width 0.05))
 (gr_line (start 144.7 128.7) (end 144.7 127.3) (layer "Edge.Cuts") (width 0.05))
 (gr_arc (start 144.7 127.3) (mid 144.787868 127.087868) (end 145 127) (layer "Edge.Cuts") (width 0.05))
 (gr_line (start 135 127) (end 128.3 127) (layer "Edge.Cuts") (width 0.05))
 (gr_line (start 145 127) (end 151.7 127) (layer "Edge.Cuts") (width 0.05))
 (gr_arc (start 127.3 157) (mid 127.087868 156.912132) (end 127 156.7) (layer "Edge.Cuts") (width 0.05))
 (gr_line (start 144.3 129) (end 144.4 129) (layer "Edge.Cuts") (width 0.05))
 (gr_arc (start 128 127.3) (mid 128.087868 127.087868) (end 128.3 127) (layer "Edge.Cuts") (width 0.05))
 (gr_line (start 128 130.2) (end 128 127.3) (layer "Edge.Cuts") (width 0.05))
 (gr_arc (start 128 130.2) (mid 127.912132 130.412132) (end 127.7 130.5) (layer "Edge.Cuts") (width 0.05))
 (gr_arc (start 127 130.8) (mid 127.087868 130.587868) (end 127.3 130.5) (layer "Edge.Cuts") (width 0.05))
 (gr_line (start 127.3 130.5) (end 127.7 130.5) (layer "Edge.Cuts") (width 0.05))
 (gr_line (start 152 130.2) (end 152 127.3) (layer "Edge.Cuts") (width 0.05))
 (gr_arc (start 152.7 130.5) (mid 152.912132 130.587868) (end 153 130.8) (layer "Edge.Cuts") (width 0.05))
 (gr_arc (start 152.3 130.5) (mid 152.087868 130.412132) (end 152 130.2) (layer "Edge.Cuts") (width 0.05))
 (gr_line (start 152.3 130.5) (end 152.7 130.5) (layer "Edge.Cuts") (width 0.05))
 (gr_line (start 127 130.8) (end 127 156.7) (layer "Edge.Cuts") (width 0.05))
 (gr_arc (start 153 156.7) (mid 152.912132 156.912132) (end 152.7 157) (layer "Edge.Cuts") (width 0.05))
 (gr_line (start 135.3 128.7) (end 135.3 127.3) (layer "Edge.Cuts") (width 0.05))
 (gr_line (start 135.6 129) (end 135.7 129) (layer "Edge.Cuts") (width 0.05))
 (gr_arc (start 151.7 127) (mid 151.912132 127.087868) (end 152 127.3) (layer "Edge.Cuts") (width 0.05))
 (gr_arc (start 135.6 129) (mid 135.387868 128.912132) (end 135.3 128.7) (layer "Edge.Cuts") (width 0.05))
 (segment (start 141.555 132.445) (end 141.4 132.6) (width 0.2) (layer "F.Cu") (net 6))
 (segment (start 141.4 132.6) (end 141.4 133.065) (width 0.2) (layer "F.Cu") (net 6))
 (segment (start 142.06 132.445) (end 141.555 132.445) (width 0.2) (layer "F.Cu") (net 6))
 (segment (start 142.51 131.75) (end 142.51 131.995) (width 0.2) (layer "F.Cu") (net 6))
 (segment (start 142.51 131.995) (end 142.06 132.445) (width 0.2) (layer "F.Cu") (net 6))
 (segment (start 141 132.5) (end 141 133.065) (width 0.2) (layer "F.Cu") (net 65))
 (segment (start 139.945 132.445) (end 140.945 132.445) (width 0.2) (layer "F.Cu") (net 65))
 (segment (start 140.945 132.445) (end 141 132.5) (width 0.2) (layer "F.Cu") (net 65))
 (segment (start 139.5 131.75) (end 139.5 132) (width 0.2) (layer "F.Cu") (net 65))
 (segment (start 139.5 132) (end 139.945 132.445) (width 0.2) (layer "F.Cu") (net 65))
 (segment (start 136.315 144.625) (end 136.315 142.387904) (width 0.25) (layer "F.Cu") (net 44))
 (segment (start 137.02 144.7) (end 136.39 144.7) (width 0.25) (layer "F.Cu") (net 44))
 (segment (start 136.39 144.7) (end 136.315 144.625) (width 0.25) (layer "F.Cu") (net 44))
 (segment (start 138.205 139.94) (end 138.2 139.935) (width 0.25) (layer "F.Cu") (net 44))
 (segment (start 138.205 140.497904) (end 138.205 139.94) (width 0.25) (layer "F.Cu") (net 44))
 (segment (start 136.315 142.387904) (end 138.205 140.497904) (width 0.25) (layer "F.Cu") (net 44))
 (segment (start 138.2 139.935) (end 138.2 139.95) (width 0.25) (layer "F.Cu") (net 44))
 (segment (start 136.35 145.35) (end 137.02 145.35) (width 0.25) (layer "F.Cu") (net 42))
 (segment (start 135.865 144.865) (end 136.35 145.35) (width 0.25) (layer "F.Cu") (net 42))
 (segment (start 137.4 139.935) (end 135.865 141.47) (width 0.25) (layer "F.Cu") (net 42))
 (segment (start 135.865 141.47) (end 135.865 144.865) (width 0.25) (layer "F.Cu") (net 42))
 (segment (start 135.415 145.051396) (end 135.415 139.585) (width 0.25) (layer "F.Cu") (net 41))
 (segment (start 137.02 146) (end 136.363604 146) (width 0.25) (layer "F.Cu") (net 41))
 (segment (start 136.363604 146) (end 135.415 145.051396) (width 0.25) (layer "F.Cu") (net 41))
 (segment (start 135.9 139.1) (end 136.565 139.1) (width 0.25) (layer "F.Cu") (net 41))
 (segment (start 135.415 139.585) (end 135.9 139.1) (width 0.25) (layer "F.Cu") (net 41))
 (segment (start 134.965 138.955) (end 135.62 138.3) (width 0.25) (layer "F.Cu") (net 39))
 (segment (start 134.965 145.237792) (end 134.965 138.955) (width 0.25) (layer "F.Cu") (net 39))
 (segment (start 136.377208 146.65) (end 134.965 145.237792) (width 0.25) (layer "F.Cu") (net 39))
 (segment (start 137.02 146.65) (end 136.377208 146.65) (width 0.25) (layer "F.Cu") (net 39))
 (segment (start 135.62 138.3) (end 136.565 138.3) (width 0.25) (layer "F.Cu") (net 39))
 (segment (start 139.75 130.448198) (end 140.52 131.218198) (width 0.2) (layer "F.Cu") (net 8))
 (segment (start 139.75 129.04) (end 139.75 130.448198) (width 0.2) (layer "F.Cu") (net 8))
 (segment (start 140.52 131.218198) (end 140.52 131.75) (width 0.2) (layer "F.Cu") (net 8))
 (segment (start 140.25 130) (end 141.49 131.24) (width 0.2) (layer "F.Cu") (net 5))
 (segment (start 140.25 129.04) (end 140.25 130) (width 0.2) (layer "F.Cu") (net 5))
 (segment (start 141.49 131.24) (end 141.49 131.75) (width 0.2) (layer "F.Cu") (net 5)))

